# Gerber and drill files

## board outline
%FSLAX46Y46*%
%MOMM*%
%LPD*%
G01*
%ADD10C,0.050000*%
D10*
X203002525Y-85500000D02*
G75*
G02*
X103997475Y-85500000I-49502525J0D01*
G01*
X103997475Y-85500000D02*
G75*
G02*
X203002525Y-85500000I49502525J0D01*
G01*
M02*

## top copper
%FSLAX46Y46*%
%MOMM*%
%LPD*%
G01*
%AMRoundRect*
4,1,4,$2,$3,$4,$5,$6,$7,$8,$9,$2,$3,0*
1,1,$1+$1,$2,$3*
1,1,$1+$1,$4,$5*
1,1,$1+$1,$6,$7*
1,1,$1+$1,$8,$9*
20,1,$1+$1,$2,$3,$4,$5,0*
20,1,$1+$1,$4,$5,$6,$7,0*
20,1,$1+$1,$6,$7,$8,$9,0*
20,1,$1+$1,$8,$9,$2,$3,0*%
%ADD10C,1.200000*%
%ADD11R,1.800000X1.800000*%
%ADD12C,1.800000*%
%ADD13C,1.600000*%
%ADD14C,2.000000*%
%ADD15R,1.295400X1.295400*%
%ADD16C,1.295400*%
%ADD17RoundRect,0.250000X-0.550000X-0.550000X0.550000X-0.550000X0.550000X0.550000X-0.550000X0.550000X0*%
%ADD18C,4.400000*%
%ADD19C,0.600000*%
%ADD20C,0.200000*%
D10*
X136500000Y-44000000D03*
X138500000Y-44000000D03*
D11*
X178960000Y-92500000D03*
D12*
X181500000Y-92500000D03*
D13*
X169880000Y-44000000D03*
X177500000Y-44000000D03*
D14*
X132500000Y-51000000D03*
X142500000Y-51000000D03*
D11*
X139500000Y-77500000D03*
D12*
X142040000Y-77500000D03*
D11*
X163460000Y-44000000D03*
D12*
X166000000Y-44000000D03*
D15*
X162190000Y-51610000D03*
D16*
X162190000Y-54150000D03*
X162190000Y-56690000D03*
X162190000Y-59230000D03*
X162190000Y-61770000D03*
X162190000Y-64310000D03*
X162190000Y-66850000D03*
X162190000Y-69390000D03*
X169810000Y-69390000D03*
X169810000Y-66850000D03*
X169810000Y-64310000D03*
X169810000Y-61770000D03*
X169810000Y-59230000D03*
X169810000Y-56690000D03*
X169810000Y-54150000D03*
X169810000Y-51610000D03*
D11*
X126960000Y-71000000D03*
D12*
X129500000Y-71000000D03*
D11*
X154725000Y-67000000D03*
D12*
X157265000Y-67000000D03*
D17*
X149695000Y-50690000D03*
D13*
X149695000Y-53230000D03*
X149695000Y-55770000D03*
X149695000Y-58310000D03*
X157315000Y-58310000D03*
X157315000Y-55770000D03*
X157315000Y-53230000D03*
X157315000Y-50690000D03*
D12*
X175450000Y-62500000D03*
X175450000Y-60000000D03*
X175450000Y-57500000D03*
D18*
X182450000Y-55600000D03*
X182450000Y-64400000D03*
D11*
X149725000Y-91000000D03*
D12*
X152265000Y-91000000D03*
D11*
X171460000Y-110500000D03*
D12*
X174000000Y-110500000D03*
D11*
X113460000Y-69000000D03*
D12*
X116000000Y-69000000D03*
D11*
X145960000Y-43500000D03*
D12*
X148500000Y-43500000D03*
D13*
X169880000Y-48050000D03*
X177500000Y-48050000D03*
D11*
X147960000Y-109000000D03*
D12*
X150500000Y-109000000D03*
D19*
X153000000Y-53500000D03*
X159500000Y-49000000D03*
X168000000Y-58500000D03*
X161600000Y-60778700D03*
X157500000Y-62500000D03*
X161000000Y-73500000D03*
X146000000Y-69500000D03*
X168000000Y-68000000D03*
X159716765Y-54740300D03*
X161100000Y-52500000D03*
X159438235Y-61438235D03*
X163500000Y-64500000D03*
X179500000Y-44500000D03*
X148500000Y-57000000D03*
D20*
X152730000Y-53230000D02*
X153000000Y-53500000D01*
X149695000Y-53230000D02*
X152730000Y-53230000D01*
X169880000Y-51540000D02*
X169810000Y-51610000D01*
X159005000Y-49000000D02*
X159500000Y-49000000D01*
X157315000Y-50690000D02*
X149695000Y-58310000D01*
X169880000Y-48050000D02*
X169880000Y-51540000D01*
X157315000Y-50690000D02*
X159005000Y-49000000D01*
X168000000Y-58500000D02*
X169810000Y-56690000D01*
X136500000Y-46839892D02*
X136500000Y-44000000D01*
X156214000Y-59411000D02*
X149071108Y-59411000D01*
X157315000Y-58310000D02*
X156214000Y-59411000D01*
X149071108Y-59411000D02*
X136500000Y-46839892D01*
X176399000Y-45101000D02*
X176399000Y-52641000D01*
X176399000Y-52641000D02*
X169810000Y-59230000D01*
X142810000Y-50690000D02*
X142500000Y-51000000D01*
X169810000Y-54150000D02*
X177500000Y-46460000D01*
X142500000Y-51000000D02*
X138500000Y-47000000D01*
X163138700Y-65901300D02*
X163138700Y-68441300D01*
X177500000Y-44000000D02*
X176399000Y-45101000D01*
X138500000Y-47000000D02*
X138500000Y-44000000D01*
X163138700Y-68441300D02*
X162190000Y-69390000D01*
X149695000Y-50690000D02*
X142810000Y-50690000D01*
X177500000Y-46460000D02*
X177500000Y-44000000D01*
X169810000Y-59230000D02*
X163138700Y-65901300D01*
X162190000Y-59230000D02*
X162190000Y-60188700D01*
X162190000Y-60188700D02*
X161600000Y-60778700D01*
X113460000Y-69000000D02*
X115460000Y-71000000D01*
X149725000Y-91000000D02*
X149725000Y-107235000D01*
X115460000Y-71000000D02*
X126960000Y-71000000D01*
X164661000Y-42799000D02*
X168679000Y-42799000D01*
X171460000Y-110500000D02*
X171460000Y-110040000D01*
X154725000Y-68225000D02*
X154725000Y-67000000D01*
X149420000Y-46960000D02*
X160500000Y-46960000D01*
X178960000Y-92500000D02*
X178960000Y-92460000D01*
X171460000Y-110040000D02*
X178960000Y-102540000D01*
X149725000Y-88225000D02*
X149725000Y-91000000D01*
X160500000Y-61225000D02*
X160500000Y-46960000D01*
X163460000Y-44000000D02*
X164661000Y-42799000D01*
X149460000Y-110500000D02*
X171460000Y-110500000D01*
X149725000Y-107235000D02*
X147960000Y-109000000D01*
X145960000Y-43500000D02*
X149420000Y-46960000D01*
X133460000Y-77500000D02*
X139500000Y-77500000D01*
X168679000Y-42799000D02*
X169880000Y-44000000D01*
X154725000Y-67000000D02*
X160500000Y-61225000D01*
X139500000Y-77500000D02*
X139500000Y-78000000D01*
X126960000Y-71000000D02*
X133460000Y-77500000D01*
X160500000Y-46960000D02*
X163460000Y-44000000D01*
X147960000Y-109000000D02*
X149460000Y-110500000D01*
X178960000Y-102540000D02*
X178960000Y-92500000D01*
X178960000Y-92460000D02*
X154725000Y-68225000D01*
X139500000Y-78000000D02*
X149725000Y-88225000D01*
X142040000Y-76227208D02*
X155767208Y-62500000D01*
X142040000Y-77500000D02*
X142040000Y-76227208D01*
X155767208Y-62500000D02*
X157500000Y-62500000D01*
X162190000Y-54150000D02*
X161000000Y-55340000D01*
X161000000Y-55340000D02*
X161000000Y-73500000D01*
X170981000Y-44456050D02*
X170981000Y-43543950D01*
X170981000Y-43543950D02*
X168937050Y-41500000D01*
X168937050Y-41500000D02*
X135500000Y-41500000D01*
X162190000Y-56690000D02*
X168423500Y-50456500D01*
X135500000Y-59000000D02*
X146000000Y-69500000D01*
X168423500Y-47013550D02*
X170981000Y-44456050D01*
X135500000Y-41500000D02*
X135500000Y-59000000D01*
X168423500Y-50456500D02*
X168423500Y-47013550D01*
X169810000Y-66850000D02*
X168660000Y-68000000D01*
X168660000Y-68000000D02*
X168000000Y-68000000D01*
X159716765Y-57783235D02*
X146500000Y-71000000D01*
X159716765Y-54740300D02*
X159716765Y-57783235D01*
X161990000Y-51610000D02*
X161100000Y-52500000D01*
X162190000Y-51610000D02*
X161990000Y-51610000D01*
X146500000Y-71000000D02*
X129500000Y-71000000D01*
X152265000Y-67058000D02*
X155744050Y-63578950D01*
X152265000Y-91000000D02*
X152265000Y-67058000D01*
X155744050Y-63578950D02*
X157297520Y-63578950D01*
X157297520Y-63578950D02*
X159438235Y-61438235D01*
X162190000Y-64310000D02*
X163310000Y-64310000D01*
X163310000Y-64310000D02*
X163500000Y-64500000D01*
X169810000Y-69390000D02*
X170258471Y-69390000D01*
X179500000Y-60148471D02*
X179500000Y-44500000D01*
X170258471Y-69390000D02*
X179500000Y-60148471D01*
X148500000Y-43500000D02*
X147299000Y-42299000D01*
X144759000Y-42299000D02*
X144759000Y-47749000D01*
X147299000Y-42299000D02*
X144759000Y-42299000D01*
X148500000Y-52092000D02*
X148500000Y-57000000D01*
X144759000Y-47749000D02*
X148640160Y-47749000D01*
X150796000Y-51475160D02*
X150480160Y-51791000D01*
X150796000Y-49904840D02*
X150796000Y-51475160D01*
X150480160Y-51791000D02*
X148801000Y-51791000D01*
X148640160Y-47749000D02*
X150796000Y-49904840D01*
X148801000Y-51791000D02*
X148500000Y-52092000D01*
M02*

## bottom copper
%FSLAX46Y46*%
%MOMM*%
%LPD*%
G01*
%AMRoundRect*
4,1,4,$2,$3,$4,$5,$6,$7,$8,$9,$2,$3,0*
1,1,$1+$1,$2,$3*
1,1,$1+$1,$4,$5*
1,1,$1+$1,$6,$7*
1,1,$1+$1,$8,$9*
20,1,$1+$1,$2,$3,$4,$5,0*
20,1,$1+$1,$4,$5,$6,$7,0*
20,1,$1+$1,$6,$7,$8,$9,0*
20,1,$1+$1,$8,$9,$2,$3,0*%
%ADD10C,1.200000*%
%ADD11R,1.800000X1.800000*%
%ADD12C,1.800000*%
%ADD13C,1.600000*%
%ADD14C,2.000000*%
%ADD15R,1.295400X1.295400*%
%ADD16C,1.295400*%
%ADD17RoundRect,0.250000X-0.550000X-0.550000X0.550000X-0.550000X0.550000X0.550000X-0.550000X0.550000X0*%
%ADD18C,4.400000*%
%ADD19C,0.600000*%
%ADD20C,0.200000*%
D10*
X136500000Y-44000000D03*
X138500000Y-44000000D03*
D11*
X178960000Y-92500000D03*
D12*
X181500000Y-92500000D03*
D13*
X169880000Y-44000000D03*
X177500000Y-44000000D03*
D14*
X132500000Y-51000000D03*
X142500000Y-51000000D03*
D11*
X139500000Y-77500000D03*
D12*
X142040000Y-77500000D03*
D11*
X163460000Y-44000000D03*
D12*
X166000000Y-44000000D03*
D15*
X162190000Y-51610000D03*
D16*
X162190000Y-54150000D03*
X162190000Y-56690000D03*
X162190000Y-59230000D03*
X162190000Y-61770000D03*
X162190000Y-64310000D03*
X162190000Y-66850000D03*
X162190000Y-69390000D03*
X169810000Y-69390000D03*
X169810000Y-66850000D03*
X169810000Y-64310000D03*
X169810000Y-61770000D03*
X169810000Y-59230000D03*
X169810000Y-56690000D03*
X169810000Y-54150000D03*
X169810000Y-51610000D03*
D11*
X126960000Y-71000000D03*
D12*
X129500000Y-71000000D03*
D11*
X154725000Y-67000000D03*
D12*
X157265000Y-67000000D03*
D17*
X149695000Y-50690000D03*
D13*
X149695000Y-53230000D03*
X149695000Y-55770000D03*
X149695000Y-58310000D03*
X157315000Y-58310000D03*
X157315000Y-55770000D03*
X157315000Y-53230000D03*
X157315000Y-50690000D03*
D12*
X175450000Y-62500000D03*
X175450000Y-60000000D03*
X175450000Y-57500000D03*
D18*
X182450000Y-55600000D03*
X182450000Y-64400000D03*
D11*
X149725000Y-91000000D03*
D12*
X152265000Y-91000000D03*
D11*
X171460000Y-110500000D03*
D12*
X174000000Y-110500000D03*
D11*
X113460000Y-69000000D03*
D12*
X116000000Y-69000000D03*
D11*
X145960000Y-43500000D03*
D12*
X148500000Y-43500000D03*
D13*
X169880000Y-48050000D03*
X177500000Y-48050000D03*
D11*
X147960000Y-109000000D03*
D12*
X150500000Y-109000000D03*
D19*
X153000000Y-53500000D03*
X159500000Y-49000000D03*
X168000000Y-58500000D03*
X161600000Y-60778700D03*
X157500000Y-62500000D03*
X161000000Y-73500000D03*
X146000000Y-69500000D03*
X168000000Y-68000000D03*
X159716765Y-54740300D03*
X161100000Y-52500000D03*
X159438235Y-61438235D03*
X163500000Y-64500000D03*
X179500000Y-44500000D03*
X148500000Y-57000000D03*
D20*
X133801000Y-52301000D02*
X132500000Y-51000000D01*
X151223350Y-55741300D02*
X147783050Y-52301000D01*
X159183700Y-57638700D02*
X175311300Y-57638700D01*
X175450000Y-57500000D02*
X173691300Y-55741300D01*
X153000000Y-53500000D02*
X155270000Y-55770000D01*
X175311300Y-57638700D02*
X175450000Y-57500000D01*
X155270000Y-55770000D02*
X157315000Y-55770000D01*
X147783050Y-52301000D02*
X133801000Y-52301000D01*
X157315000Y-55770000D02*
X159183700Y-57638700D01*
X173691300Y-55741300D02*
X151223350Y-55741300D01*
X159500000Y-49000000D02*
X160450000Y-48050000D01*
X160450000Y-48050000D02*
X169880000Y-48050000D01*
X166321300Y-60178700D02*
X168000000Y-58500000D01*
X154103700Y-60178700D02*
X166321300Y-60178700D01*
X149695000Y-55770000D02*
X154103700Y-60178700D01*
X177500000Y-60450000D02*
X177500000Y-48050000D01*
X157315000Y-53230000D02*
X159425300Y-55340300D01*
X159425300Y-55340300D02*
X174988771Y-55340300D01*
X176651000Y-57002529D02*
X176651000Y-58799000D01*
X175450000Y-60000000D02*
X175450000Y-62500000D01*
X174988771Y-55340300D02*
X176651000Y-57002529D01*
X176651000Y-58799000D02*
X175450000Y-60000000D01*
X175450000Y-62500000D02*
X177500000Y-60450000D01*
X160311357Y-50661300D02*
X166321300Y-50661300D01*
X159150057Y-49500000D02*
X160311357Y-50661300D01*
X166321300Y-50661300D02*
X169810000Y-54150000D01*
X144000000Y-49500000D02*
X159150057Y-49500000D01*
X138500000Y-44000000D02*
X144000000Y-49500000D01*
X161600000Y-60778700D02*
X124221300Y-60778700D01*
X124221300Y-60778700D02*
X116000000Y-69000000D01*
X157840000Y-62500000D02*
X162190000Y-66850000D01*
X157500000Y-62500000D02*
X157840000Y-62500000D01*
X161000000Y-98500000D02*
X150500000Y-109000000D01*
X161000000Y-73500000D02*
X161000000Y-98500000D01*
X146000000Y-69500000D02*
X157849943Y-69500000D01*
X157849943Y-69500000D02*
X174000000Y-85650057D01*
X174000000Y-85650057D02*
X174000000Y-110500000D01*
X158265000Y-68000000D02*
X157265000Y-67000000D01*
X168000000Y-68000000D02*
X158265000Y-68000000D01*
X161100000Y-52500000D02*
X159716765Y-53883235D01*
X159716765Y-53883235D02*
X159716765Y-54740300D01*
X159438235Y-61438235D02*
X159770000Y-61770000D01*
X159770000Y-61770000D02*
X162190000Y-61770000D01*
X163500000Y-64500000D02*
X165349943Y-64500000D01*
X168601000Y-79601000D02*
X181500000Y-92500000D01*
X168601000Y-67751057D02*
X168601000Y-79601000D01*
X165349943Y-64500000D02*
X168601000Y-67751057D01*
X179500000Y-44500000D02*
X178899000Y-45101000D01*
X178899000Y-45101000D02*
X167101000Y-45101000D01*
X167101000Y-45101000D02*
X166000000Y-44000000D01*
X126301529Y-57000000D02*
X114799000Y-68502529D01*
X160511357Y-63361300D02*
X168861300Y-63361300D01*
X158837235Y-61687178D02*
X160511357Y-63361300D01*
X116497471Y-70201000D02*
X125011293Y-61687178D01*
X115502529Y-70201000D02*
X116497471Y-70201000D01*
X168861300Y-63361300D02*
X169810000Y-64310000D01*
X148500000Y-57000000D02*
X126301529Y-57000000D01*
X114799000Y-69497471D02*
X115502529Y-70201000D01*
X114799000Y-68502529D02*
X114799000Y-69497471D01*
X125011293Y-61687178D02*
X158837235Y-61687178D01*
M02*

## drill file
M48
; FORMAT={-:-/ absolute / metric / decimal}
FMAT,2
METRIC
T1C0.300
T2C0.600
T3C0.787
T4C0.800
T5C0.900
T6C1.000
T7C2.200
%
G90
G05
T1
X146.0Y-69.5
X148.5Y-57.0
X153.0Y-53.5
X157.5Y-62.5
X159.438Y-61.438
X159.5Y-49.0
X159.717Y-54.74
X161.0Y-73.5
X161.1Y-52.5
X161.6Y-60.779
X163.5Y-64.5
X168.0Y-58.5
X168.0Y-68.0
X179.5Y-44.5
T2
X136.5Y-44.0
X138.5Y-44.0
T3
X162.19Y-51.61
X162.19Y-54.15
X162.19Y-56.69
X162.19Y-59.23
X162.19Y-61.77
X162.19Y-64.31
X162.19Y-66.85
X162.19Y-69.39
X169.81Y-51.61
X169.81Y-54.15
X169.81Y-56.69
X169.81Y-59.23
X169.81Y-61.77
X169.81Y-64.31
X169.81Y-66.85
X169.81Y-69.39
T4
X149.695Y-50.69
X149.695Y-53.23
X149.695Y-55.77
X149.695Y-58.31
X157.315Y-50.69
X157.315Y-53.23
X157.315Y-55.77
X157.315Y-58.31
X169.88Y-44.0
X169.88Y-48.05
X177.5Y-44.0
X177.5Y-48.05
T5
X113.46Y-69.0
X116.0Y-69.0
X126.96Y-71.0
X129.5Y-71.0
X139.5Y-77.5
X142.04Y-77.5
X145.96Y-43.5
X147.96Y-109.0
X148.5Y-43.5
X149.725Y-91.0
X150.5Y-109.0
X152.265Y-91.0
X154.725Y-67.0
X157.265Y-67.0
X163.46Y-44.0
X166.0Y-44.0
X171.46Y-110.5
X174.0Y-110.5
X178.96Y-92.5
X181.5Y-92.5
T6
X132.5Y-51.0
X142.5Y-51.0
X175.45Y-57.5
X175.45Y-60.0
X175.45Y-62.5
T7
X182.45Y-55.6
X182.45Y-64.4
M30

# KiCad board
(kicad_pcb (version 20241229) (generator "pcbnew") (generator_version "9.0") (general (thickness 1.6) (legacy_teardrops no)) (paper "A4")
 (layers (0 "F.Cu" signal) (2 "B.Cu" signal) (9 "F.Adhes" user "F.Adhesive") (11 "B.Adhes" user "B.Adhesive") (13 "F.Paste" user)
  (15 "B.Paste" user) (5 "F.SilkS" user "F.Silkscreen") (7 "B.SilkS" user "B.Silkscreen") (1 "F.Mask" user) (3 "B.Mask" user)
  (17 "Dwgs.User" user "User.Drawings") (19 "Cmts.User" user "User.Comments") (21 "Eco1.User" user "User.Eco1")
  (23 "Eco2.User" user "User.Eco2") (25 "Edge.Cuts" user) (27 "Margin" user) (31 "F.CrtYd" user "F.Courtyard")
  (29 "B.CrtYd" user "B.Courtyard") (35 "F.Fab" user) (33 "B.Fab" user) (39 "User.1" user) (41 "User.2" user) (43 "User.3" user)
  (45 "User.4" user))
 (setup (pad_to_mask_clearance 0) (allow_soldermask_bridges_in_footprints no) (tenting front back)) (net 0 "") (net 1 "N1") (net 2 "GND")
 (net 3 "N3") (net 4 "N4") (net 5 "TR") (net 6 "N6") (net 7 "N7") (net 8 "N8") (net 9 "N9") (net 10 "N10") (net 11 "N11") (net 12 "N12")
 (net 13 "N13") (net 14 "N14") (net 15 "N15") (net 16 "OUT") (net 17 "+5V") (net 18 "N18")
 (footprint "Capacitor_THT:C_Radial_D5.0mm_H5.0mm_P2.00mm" (layer "F.Cu") (at 136.5 44)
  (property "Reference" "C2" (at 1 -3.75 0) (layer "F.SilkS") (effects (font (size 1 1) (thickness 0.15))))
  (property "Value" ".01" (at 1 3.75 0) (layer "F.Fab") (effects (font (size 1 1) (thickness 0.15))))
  (pad "1" thru_hole circle (at 0 0) (size 1.2 1.2) (drill 0.6) (layers "*.Cu" "*.Mask") (remove_unused_layers no) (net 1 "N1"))
  (pad "2" thru_hole circle (at 2 0) (size 1.2 1.2) (drill 0.6) (layers "*.Cu" "*.Mask") (remove_unused_layers no) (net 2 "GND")))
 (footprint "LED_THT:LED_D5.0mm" (layer "F.Cu") (at 178.96 92.5)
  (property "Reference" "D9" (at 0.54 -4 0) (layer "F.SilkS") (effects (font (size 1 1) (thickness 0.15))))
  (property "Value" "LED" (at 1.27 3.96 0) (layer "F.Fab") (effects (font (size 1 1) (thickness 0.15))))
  (pad "1" thru_hole rect (at 0 0) (size 1.8 1.8) (drill 0.9) (layers "*.Cu" "*.Mask") (remove_unused_layers no) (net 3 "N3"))
  (pad "2" thru_hole circle (at 2.54 0) (size 1.8 1.8) (drill 0.9) (layers "*.Cu" "*.Mask") (remove_unused_layers no) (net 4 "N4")))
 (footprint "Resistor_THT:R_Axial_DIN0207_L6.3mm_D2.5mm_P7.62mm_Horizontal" (layer "F.Cu") (at 169.88 44)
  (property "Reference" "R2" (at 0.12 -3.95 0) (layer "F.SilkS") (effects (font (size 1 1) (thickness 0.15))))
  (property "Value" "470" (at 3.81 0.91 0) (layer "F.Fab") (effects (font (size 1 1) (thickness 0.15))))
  (pad "1" thru_hole circle (at 0 0) (size 1.6 1.6) (drill 0.8) (layers "*.Cu" "*.Mask") (remove_unused_layers no) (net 3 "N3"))
  (pad "2" thru_hole circle (at 7.62 0) (size 1.6 1.6) (drill 0.8) (layers "*.Cu" "*.Mask") (remove_unused_layers no) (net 2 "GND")))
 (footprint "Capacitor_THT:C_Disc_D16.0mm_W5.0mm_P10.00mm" (layer "F.Cu") (at 132.5 51)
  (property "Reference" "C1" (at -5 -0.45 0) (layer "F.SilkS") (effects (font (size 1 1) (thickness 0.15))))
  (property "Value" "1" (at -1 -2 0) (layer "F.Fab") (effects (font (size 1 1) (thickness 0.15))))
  (pad "1" thru_hole circle (at 0 0) (size 2 2) (drill 1) (layers "*.Cu" "*.Mask") (remove_unused_layers no) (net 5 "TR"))
  (pad "2" thru_hole circle (at 10 0) (size 2 2) (drill 1) (layers "*.Cu" "*.Mask") (remove_unused_layers no) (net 2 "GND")))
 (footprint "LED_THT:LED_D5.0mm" (layer "F.Cu") (at 139.5 77.5)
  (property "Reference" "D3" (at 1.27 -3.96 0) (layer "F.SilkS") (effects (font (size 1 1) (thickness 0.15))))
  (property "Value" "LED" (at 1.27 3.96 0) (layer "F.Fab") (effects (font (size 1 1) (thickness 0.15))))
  (pad "1" thru_hole rect (at 0 0) (size 1.8 1.8) (drill 0.9) (layers "*.Cu" "*.Mask") (remove_unused_layers no) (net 3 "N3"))
  (pad "2" thru_hole circle (at 2.54 0) (size 1.8 1.8) (drill 0.9) (layers "*.Cu" "*.Mask") (remove_unused_layers no) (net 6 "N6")))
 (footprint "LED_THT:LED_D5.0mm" (layer "F.Cu") (at 163.46 44)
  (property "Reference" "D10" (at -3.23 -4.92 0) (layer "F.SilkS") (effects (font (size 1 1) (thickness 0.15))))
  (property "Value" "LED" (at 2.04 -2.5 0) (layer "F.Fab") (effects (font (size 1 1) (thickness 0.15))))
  (pad "1" thru_hole rect (at 0 0) (size 1.8 1.8) (drill 0.9) (layers "*.Cu" "*.Mask") (remove_unused_layers no) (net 3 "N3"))
  (pad "2" thru_hole circle (at 2.54 0) (size 1.8 1.8) (drill 0.9) (layers "*.Cu" "*.Mask") (remove_unused_layers no) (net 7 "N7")))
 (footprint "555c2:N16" (layer "F.Cu") (at 169.81 69.39)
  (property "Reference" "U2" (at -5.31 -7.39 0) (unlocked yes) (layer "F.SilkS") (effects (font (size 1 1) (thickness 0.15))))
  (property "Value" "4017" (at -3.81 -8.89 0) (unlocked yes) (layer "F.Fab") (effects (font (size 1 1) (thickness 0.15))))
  (pad "1" thru_hole rect (at -7.62 -17.78) (size 1.2954 1.2954) (drill 0.7874) (layers "*.Cu" "*.Mask") (remove_unused_layers no)
   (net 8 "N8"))
  (pad "2" thru_hole circle (at -7.62 -15.24) (size 1.2954 1.2954) (drill 0.7874) (layers "*.Cu" "*.Mask") (remove_unused_layers no)
   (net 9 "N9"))
  (pad "3" thru_hole circle (at -7.62 -12.7) (size 1.2954 1.2954) (drill 0.7874) (layers "*.Cu" "*.Mask") (remove_unused_layers no)
   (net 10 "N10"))
  (pad "4" thru_hole circle (at -7.62 -10.16) (size 1.2954 1.2954) (drill 0.7874) (layers "*.Cu" "*.Mask") (remove_unused_layers no)
   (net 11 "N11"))
  (pad "5" thru_hole circle (at -7.62 -7.62) (size 1.2954 1.2954) (drill 0.7874) (layers "*.Cu" "*.Mask") (remove_unused_layers no)
   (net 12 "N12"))
  (pad "6" thru_hole circle (at -7.62 -5.08) (size 1.2954 1.2954) (drill 0.7874) (layers "*.Cu" "*.Mask") (remove_unused_layers no)
   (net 4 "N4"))
  (pad "7" thru_hole circle (at -7.62 -2.54) (size 1.2954 1.2954) (drill 0.7874) (layers "*.Cu" "*.Mask") (remove_unused_layers no)
   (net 6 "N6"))
  (pad "8" thru_hole circle (at -7.62 0) (size 1.2954 1.2954) (drill 0.7874) (layers "*.Cu" "*.Mask") (remove_unused_layers no)
   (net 2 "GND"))
  (pad "9" thru_hole circle (at 0 0) (size 1.2954 1.2954) (drill 0.7874) (layers "*.Cu" "*.Mask") (remove_unused_layers no) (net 7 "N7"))
  (pad "10" thru_hole circle (at 0 -2.54) (size 1.2954 1.2954) (drill 0.7874) (layers "*.Cu" "*.Mask") (remove_unused_layers no)
   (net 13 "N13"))
  (pad "11" thru_hole circle (at 0 -5.08) (size 1.2954 1.2954) (drill 0.7874) (layers "*.Cu" "*.Mask") (remove_unused_layers no)
   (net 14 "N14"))
  (pad "12" thru_hole circle (at 0 -7.62) (size 1.2954 1.2954) (drill 0.7874) (layers "*.Cu" "*.Mask") (remove_unused_layers no)
   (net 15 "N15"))
  (pad "13" thru_hole circle (at 0 -10.16) (size 1.2954 1.2954) (drill 0.7874) (layers "*.Cu" "*.Mask") (remove_unused_layers no)
   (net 2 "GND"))
  (pad "14" thru_hole circle (at 0 -12.7) (size 1.2954 1.2954) (drill 0.7874) (layers "*.Cu" "*.Mask") (remove_unused_layers no)
   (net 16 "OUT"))
  (pad "15" thru_hole circle (at 0 -15.24) (size 1.2954 1.2954) (drill 0.7874) (layers "*.Cu" "*.Mask") (remove_unused_layers no)
   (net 2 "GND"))
  (pad "16" thru_hole circle (at 0 -17.78) (size 1.2954 1.2954) (drill 0.7874) (layers "*.Cu" "*.Mask") (remove_unused_layers no)
   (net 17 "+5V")))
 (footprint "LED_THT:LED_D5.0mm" (layer "F.Cu") (at 126.96 71)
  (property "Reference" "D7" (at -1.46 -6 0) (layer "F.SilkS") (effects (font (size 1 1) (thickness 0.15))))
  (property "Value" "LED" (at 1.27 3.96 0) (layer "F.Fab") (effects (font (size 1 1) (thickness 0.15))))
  (pad "1" thru_hole rect (at 0 0) (size 1.8 1.8) (drill 0.9) (layers "*.Cu" "*.Mask") (remove_unused_layers no) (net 3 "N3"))
  (pad "2" thru_hole circle (at 2.54 0) (size 1.8 1.8) (drill 0.9) (layers "*.Cu" "*.Mask") (remove_unused_layers no) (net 8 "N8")))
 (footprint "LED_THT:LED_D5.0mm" (layer "F.Cu") (at 154.725 67)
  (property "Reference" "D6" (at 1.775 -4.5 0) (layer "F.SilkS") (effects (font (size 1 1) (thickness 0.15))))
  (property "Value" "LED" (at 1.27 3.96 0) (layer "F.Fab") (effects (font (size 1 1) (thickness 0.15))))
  (pad "1" thru_hole rect (at 0 0) (size 1.8 1.8) (drill 0.9) (layers "*.Cu" "*.Mask") (remove_unused_layers no) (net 3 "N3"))
  (pad "2" thru_hole circle (at 2.54 0) (size 1.8 1.8) (drill 0.9) (layers "*.Cu" "*.Mask") (remove_unused_layers no) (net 13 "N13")))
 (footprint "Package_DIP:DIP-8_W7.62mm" (layer "F.Cu") (at 149.695 50.69)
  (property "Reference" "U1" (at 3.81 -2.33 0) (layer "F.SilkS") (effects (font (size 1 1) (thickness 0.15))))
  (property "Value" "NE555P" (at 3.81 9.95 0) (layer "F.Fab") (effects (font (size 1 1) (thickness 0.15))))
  (pad "1" thru_hole roundrect (at 0 0) (size 1.6 1.6) (drill 0.8) (layers "*.Cu" "*.Mask") (remove_unused_layers no)
   (roundrect_rratio 0.15625) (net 2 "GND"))
  (pad "2" thru_hole circle (at 0 2.54) (size 1.6 1.6) (drill 0.8) (layers "*.Cu" "*.Mask") (remove_unused_layers no) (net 5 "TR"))
  (pad "3" thru_hole circle (at 0 5.08) (size 1.6 1.6) (drill 0.8) (layers "*.Cu" "*.Mask") (remove_unused_layers no) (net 16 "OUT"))
  (pad "4" thru_hole circle (at 0 7.62) (size 1.6 1.6) (drill 0.8) (layers "*.Cu" "*.Mask") (remove_unused_layers no) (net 17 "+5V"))
  (pad "5" thru_hole circle (at 7.62 7.62) (size 1.6 1.6) (drill 0.8) (layers "*.Cu" "*.Mask") (remove_unused_layers no) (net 1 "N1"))
  (pad "6" thru_hole circle (at 7.62 5.08) (size 1.6 1.6) (drill 0.8) (layers "*.Cu" "*.Mask") (remove_unused_layers no) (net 5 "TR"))
  (pad "7" thru_hole circle (at 7.62 2.54) (size 1.6 1.6) (drill 0.8) (layers "*.Cu" "*.Mask") (remove_unused_layers no) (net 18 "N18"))
  (pad "8" thru_hole circle (at 7.62 0) (size 1.6 1.6) (drill 0.8) (layers "*.Cu" "*.Mask") (remove_unused_layers no) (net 17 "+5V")))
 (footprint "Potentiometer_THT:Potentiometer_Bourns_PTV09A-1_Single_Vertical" (layer "F.Cu") (at 175.45 62.5)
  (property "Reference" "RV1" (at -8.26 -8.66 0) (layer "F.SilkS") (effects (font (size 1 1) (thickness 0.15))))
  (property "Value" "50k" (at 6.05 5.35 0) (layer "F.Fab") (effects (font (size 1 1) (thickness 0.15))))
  (pad "1" thru_hole circle (at 0 0) (size 1.8 1.8) (drill 1) (layers "*.Cu" "*.Mask") (remove_unused_layers no) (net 18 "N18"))
  (pad "2" thru_hole circle (at 0 -2.5) (size 1.8 1.8) (drill 1) (layers "*.Cu" "*.Mask") (remove_unused_layers no) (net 18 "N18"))
  (pad "3" thru_hole circle (at 0 -5) (size 1.8 1.8) (drill 1) (layers "*.Cu" "*.Mask") (remove_unused_layers no) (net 5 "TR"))
  (pad "MP" thru_hole circle (at 7 -6.9) (size 4.4 4.4) (drill 2.2) (layers "*.Cu" "*.Mask") (remove_unused_layers no))
  (pad "MP" thru_hole circle (at 7 1.9) (size 4.4 4.4) (drill 2.2) (layers "*.Cu" "*.Mask") (remove_unused_layers no)))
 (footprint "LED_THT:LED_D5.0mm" (layer "F.Cu") (at 149.725 91)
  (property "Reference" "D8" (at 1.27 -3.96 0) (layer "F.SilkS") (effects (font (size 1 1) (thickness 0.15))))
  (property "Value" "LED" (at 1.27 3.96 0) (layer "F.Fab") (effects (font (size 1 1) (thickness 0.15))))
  (pad "1" thru_hole rect (at 0 0) (size 1.8 1.8) (drill 0.9) (layers "*.Cu" "*.Mask") (remove_unused_layers no) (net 3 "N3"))
  (pad "2" thru_hole circle (at 2.54 0) (size 1.8 1.8) (drill 0.9) (layers "*.Cu" "*.Mask") (remove_unused_layers no) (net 12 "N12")))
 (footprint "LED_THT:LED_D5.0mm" (layer "F.Cu") (at 171.46 110.5)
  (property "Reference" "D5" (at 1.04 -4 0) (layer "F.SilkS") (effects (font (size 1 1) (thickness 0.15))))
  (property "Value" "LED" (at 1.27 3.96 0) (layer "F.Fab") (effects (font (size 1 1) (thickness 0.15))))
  (pad "1" thru_hole rect (at 0 0) (size 1.8 1.8) (drill 0.9) (layers "*.Cu" "*.Mask") (remove_unused_layers no) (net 3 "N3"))
  (pad "2" thru_hole circle (at 2.54 0) (size 1.8 1.8) (drill 0.9) (layers "*.Cu" "*.Mask") (remove_unused_layers no) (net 10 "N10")))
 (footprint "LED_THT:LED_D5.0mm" (layer "F.Cu") (at 113.46 69)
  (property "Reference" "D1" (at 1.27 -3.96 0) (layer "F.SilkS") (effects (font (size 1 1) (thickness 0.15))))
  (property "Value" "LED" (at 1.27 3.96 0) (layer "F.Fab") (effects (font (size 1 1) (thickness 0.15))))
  (pad "1" thru_hole rect (at 0 0) (size 1.8 1.8) (drill 0.9) (layers "*.Cu" "*.Mask") (remove_unused_layers no) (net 3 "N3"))
  (pad "2" thru_hole circle (at 2.54 0) (size 1.8 1.8) (drill 0.9) (layers "*.Cu" "*.Mask") (remove_unused_layers no) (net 11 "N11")))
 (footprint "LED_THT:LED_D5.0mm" (layer "F.Cu") (at 145.96 43.5)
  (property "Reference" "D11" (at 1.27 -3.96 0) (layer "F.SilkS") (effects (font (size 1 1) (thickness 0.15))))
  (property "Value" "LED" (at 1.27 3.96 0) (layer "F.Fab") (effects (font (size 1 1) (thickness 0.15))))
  (pad "1" thru_hole rect (at 0 0) (size 1.8 1.8) (drill 0.9) (layers "*.Cu" "*.Mask") (remove_unused_layers no) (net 3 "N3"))
  (pad "2" thru_hole circle (at 2.54 0) (size 1.8 1.8) (drill 0.9) (layers "*.Cu" "*.Mask") (remove_unused_layers no) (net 14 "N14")))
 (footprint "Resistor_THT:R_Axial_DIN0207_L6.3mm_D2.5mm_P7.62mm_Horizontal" (layer "F.Cu") (at 169.88 48.05)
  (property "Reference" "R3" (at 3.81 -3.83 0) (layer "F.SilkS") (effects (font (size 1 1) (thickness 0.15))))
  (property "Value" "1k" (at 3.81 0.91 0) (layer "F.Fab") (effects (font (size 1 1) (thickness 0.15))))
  (pad "1" thru_hole circle (at 0 0) (size 1.6 1.6) (drill 0.8) (layers "*.Cu" "*.Mask") (remove_unused_layers no) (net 17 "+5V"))
  (pad "2" thru_hole circle (at 7.62 0) (size 1.6 1.6) (drill 0.8) (layers "*.Cu" "*.Mask") (remove_unused_layers no) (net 18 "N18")))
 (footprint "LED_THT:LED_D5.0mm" (layer "F.Cu") (at 147.96 109)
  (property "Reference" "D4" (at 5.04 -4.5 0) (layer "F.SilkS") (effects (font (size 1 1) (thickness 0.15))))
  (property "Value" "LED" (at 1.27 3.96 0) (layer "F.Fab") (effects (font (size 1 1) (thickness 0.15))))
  (pad "1" thru_hole rect (at 0 0) (size 1.8 1.8) (drill 0.9) (layers "*.Cu" "*.Mask") (remove_unused_layers no) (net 3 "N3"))
  (pad "2" thru_hole circle (at 2.54 0) (size 1.8 1.8) (drill 0.9) (layers "*.Cu" "*.Mask") (remove_unused_layers no) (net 9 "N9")))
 (gr_circle (center 153.5 85.5) (end 119 50) (stroke (width 0.05) (type default)) (fill no) (layer "Edge.Cuts"))
 (segment (start 152.73 53.23) (end 153 53.5) (width 0.2) (layer "F.Cu") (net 5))
 (segment (start 149.695 53.23) (end 152.73 53.23) (width 0.2) (layer "F.Cu") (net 5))
 (via (at 153 53.5) (size 0.6) (drill 0.3) (layers "F.Cu" "B.Cu") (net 5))
 (segment (start 133.801 52.301) (end 132.5 51) (width 0.2) (layer "B.Cu") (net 5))
 (segment (start 151.22335 55.7413) (end 147.78305 52.301) (width 0.2) (layer "B.Cu") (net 5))
 (segment (start 159.1837 57.6387) (end 175.3113 57.6387) (width 0.2) (layer "B.Cu") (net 5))
 (segment (start 175.45 57.5) (end 173.6913 55.7413) (width 0.2) (layer "B.Cu") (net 5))
 (segment (start 153 53.5) (end 155.27 55.77) (width 0.2) (layer "B.Cu") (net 5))
 (segment (start 175.3113 57.6387) (end 175.45 57.5) (width 0.2) (layer "B.Cu") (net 5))
 (segment (start 155.27 55.77) (end 157.315 55.77) (width 0.2) (layer "B.Cu") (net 5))
 (segment (start 147.78305 52.301) (end 133.801 52.301) (width 0.2) (layer "B.Cu") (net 5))
 (segment (start 157.315 55.77) (end 159.1837 57.6387) (width 0.2) (layer "B.Cu") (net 5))
 (segment (start 173.6913 55.7413) (end 151.22335 55.7413) (width 0.2) (layer "B.Cu") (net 5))
 (segment (start 169.88 51.54) (end 169.81 51.61) (width 0.2) (layer "F.Cu") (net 17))
 (segment (start 159.005 49) (end 159.5 49) (width 0.2) (layer "F.Cu") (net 17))
 (segment (start 157.315 50.69) (end 149.695 58.31) (width 0.2) (layer "F.Cu") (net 17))
 (segment (start 169.88 48.05) (end 169.88 51.54) (width 0.2) (layer "F.Cu") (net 17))
 (segment (start 157.315 50.69) (end 159.005 49) (width 0.2) (layer "F.Cu") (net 17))
 (via (at 159.5 49) (size 0.6) (drill 0.3) (layers "F.Cu" "B.Cu") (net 17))
 (segment (start 159.5 49) (end 160.45 48.05) (width 0.2) (layer "B.Cu") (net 17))
 (segment (start 160.45 48.05) (end 169.88 48.05) (width 0.2) (layer "B.Cu") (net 17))
 (segment (start 168 58.5) (end 169.81 56.69) (width 0.2) (layer "F.Cu") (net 16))
 (via (at 168 58.5) (size 0.6) (drill 0.3) (layers "F.Cu" "B.Cu") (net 16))
 (segment (start 166.3213 60.1787) (end 168 58.5) (width 0.2) (layer "B.Cu") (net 16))
 (segment (start 154.1037 60.1787) (end 166.3213 60.1787) (width 0.2) (layer "B.Cu") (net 16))
 (segment (start 149.695 55.77) (end 154.1037 60.1787) (width 0.2) (layer "B.Cu") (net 16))
 (segment (start 136.5 46.839892) (end 136.5 44) (width 0.2) (layer "F.Cu") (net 1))
 (segment (start 156.214 59.411) (end 149.071108 59.411) (width 0.2) (layer "F.Cu") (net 1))
 (segment (start 157.315 58.31) (end 156.214 59.411) (width 0.2) (layer "F.Cu") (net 1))
 (segment (start 149.071108 59.411) (end 136.5 46.839892) (width 0.2) (layer "F.Cu") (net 1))
 (segment (start 177.5 60.45) (end 177.5 48.05) (width 0.2) (layer "B.Cu") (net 18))
 (segment (start 157.315 53.23) (end 159.4253 55.3403) (width 0.2) (layer "B.Cu") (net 18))
 (segment (start 159.4253 55.3403) (end 174.988771 55.3403) (width 0.2) (layer "B.Cu") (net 18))
 (segment (start 176.651 57.002529) (end 176.651 58.799) (width 0.2) (layer "B.Cu") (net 18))
 (segment (start 175.45 60) (end 175.45 62.5) (width 0.2) (layer "B.Cu") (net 18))
 (segment (start 174.988771 55.3403) (end 176.651 57.002529) (width 0.2) (layer "B.Cu") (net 18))
 (segment (start 176.651 58.799) (end 175.45 60) (width 0.2) (layer "B.Cu") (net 18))
 (segment (start 175.45 62.5) (end 177.5 60.45) (width 0.2) (layer "B.Cu") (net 18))
 (segment (start 176.399 45.101) (end 176.399 52.641) (width 0.2) (layer "F.Cu") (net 2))
 (segment (start 176.399 52.641) (end 169.81 59.23) (width 0.2) (layer "F.Cu") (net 2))
 (segment (start 142.81 50.69) (end 142.5 51) (width 0.2) (layer "F.Cu") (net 2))
 (segment (start 169.81 54.15) (end 177.5 46.46) (width 0.2) (layer "F.Cu") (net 2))
 (segment (start 142.5 51) (end 138.5 47) (width 0.2) (layer "F.Cu") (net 2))
 (segment (start 163.1387 65.9013) (end 163.1387 68.4413) (width 0.2) (layer "F.Cu") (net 2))
 (segment (start 177.5 44) (end 176.399 45.101) (width 0.2) (layer "F.Cu") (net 2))
 (segment (start 138.5 47) (end 138.5 44) (width 0.2) (layer "F.Cu") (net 2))
 (segment (start 163.1387 68.4413) (end 162.19 69.39) (width 0.2) (layer "F.Cu") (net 2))
 (segment (start 149.695 50.69) (end 142.81 50.69) (width 0.2) (layer "F.Cu") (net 2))
 (segment (start 177.5 46.46) (end 177.5 44) (width 0.2) (layer "F.Cu") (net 2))
 (segment (start 169.81 59.23) (end 163.1387 65.9013) (width 0.2) (layer "F.Cu") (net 2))
 (segment (start 160.311357 50.6613) (end 166.3213 50.6613) (width 0.2) (layer "B.Cu") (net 2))
 (segment (start 159.150057 49.5) (end 160.311357 50.6613) (width 0.2) (layer "B.Cu") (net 2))
 (segment (start 166.3213 50.6613) (end 169.81 54.15) (width 0.2) (layer "B.Cu") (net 2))
 (segment (start 144 49.5) (end 159.150057 49.5) (width 0.2) (layer "B.Cu") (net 2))
 (segment (start 138.5 44) (end 144 49.5) (width 0.2) (layer "B.Cu") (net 2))
 (segment (start 162.19 59.23) (end 162.19 60.1887) (width 0.2) (layer "F.Cu") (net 11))
 (segment (start 162.19 60.1887) (end 161.6 60.7787) (width 0.2) (layer "F.Cu") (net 11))
 (via (at 161.6 60.7787) (size 0.6) (drill 0.3) (layers "F.Cu" "B.Cu") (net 11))
 (segment (start 161.6 60.7787) (end 124.2213 60.7787) (width 0.2) (layer "B.Cu") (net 11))
 (segment (start 124.2213 60.7787) (end 116 69) (width 0.2) (layer "B.Cu") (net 11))
 (segment (start 113.46 69) (end 115.46 71) (width 0.2) (layer "F.Cu") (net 3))
 (segment (start 149.725 91) (end 149.725 107.235) (width 0.2) (layer "F.Cu") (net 3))
 (segment (start 115.46 71) (end 126.96 71) (width 0.2) (layer "F.Cu") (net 3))
 (segment (start 164.661 42.799) (end 168.679 42.799) (width 0.2) (layer "F.Cu") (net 3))
 (segment (start 171.46 110.5) (end 171.46 110.04) (width 0.2) (layer "F.Cu") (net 3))
 (segment (start 154.725 68.225) (end 154.725 67) (width 0.2) (layer "F.Cu") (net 3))
 (segment (start 149.42 46.96) (end 160.5 46.96) (width 0.2) (layer "F.Cu") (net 3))
 (segment (start 178.96 92.5) (end 178.96 92.46) (width 0.2) (layer "F.Cu") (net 3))
 (segment (start 171.46 110.04) (end 178.96 102.54) (width 0.2) (layer "F.Cu") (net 3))
 (segment (start 149.725 88.225) (end 149.725 91) (width 0.2) (layer "F.Cu") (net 3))
 (segment (start 160.5 61.225) (end 160.5 46.96) (width 0.2) (layer "F.Cu") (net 3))
 (segment (start 163.46 44) (end 164.661 42.799) (width 0.2) (layer "F.Cu") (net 3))
 (segment (start 149.46 110.5) (end 171.46 110.5) (width 0.2) (layer "F.Cu") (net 3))
 (segment (start 149.725 107.235) (end 147.96 109) (width 0.2) (layer "F.Cu") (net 3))
 (segment (start 145.96 43.5) (end 149.42 46.96) (width 0.2) (layer "F.Cu") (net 3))
 (segment (start 133.46 77.5) (end 139.5 77.5) (width 0.2) (layer "F.Cu") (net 3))
 (segment (start 168.679 42.799) (end 169.88 44) (width 0.2) (layer "F.Cu") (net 3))
 (segment (start 154.725 67) (end 160.5 61.225) (width 0.2) (layer "F.Cu") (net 3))
 (segment (start 139.5 77.5) (end 139.5 78) (width 0.2) (layer "F.Cu") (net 3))
 (segment (start 126.96 71) (end 133.46 77.5) (width 0.2) (layer "F.Cu") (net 3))
 (segment (start 160.5 46.96) (end 163.46 44) (width 0.2) (layer "F.Cu") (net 3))
 (segment (start 147.96 109) (end 149.46 110.5) (width 0.2) (layer "F.Cu") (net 3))
 (segment (start 178.96 102.54) (end 178.96 92.5) (width 0.2) (layer "F.Cu") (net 3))
 (segment (start 178.96 92.46) (end 154.725 68.225) (width 0.2) (layer "F.Cu") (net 3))
 (segment (start 139.5 78) (end 149.725 88.225) (width 0.2) (layer "F.Cu") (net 3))
 (segment (start 142.04 76.227208) (end 155.767208 62.5) (width 0.2) (layer "F.Cu") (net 6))
 (segment (start 142.04 77.5) (end 142.04 76.227208) (width 0.2) (layer "F.Cu") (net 6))
 (segment (start 155.767208 62.5) (end 157.5 62.5) (width 0.2) (layer "F.Cu") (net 6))
 (via (at 157.5 62.5) (size 0.6) (drill 0.3) (layers "F.Cu" "B.Cu") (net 6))
 (segment (start 157.84 62.5) (end 162.19 66.85) (width 0.2) (layer "B.Cu") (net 6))
 (segment (start 157.5 62.5) (end 157.84 62.5) (width 0.2) (layer "B.Cu") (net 6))
 (segment (start 162.19 54.15) (end 161 55.34) (width 0.2) (layer "F.Cu") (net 9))
 (segment (start 161 55.34) (end 161 73.5) (width 0.2) (layer "F.Cu") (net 9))
 (via (at 161 73.5) (size 0.6) (drill 0.3) (layers "F.Cu" "B.Cu") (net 9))
 (segment (start 161 98.5) (end 150.5 109) (width 0.2) (layer "B.Cu") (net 9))
 (segment (start 161 73.5) (end 161 98.5) (width 0.2) (layer "B.Cu") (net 9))
 (segment (start 170.981 44.45605) (end 170.981 43.54395) (width 0.2) (layer "F.Cu") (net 10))
 (segment (start 170.981 43.54395) (end 168.93705 41.5) (width 0.2) (layer "F.Cu") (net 10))
 (segment (start 168.93705 41.5) (end 135.5 41.5) (width 0.2) (layer "F.Cu") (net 10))
 (segment (start 162.19 56.69) (end 168.4235 50.4565) (width 0.2) (layer "F.Cu") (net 10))
 (segment (start 135.5 59) (end 146 69.5) (width 0.2) (layer "F.Cu") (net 10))
 (segment (start 168.4235 47.01355) (end 170.981 44.45605) (width 0.2) (layer "F.Cu") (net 10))
 (segment (start 135.5 41.5) (end 135.5 59) (width 0.2) (layer "F.Cu") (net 10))
 (segment (start 168.4235 50.4565) (end 168.4235 47.01355) (width 0.2) (layer "F.Cu") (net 10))
 (via (at 146 69.5) (size 0.6) (drill 0.3) (layers "F.Cu" "B.Cu") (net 10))
 (segment (start 146 69.5) (end 157.849943 69.5) (width 0.2) (layer "B.Cu") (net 10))
 (segment (start 157.849943 69.5) (end 174 85.650057) (width 0.2) (layer "B.Cu") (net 10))
 (segment (start 174 85.650057) (end 174 110.5) (width 0.2) (layer "B.Cu") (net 10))
 (segment (start 169.81 66.85) (end 168.66 68) (width 0.2) (layer "F.Cu") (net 13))
 (segment (start 168.66 68) (end 168 68) (width 0.2) (layer "F.Cu") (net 13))
 (via (at 168 68) (size 0.6) (drill 0.3) (layers "F.Cu" "B.Cu") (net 13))
 (segment (start 158.265 68) (end 157.265 67) (width 0.2) (layer "B.Cu") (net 13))
 (segment (start 168 68) (end 158.265 68) (width 0.2) (layer "B.Cu") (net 13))
 (segment (start 159.716765 57.783235) (end 146.5 71) (width 0.2) (layer "F.Cu") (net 8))
 (segment (start 159.716765 54.7403) (end 159.716765 57.783235) (width 0.2) (layer "F.Cu") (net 8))
 (segment (start 161.99 51.61) (end 161.1 52.5) (width 0.2) (layer "F.Cu") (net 8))
 (segment (start 162.19 51.61) (end 161.99 51.61) (width 0.2) (layer "F.Cu") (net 8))
 (segment (start 146.5 71) (end 129.5 71) (width 0.2) (layer "F.Cu") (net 8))
 (via (at 159.716765 54.7403) (size 0.6) (drill 0.3) (layers "F.Cu" "B.Cu") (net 8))
 (via (at 161.1 52.5) (size 0.6) (drill 0.3) (layers "F.Cu" "B.Cu") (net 8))
 (segment (start 161.1 52.5) (end 159.716765 53.883235) (width 0.2) (layer "B.Cu") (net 8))
 (segment (start 159.716765 53.883235) (end 159.716765 54.7403) (width 0.2) (layer "B.Cu") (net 8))
 (segment (start 152.265 67.058) (end 155.74405 63.57895) (width 0.2) (layer "F.Cu") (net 12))
 (segment (start 152.265 91) (end 152.265 67.058) (width 0.2) (layer "F.Cu") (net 12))
 (segment (start 155.74405 63.57895) (end 157.29752 63.57895) (width 0.2) (layer "F.Cu") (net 12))
 (segment (start 157.29752 63.57895) (end 159.438235 61.438235) (width 0.2) (layer "F.Cu") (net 12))
 (via (at 159.438235 61.438235) (size 0.6) (drill 0.3) (layers "F.Cu" "B.Cu") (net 12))
 (segment (start 159.438235 61.438235) (end 159.77 61.77) (width 0.2) (layer "B.Cu") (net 12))
 (segment (start 159.77 61.77) (end 162.19 61.77) (width 0.2) (layer "B.Cu") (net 12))
 (segment (start 162.19 64.31) (end 163.31 64.31) (width 0.2) (layer "F.Cu") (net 4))
 (segment (start 163.31 64.31) (end 163.5 64.5) (width 0.2) (layer "F.Cu") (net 4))
 (via (at 163.5 64.5) (size 0.6) (drill 0.3) (layers "F.Cu" "B.Cu") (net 4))
 (segment (start 163.5 64.5) (end 165.349943 64.5) (width 0.2) (layer "B.Cu") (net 4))
 (segment (start 168.601 79.601) (end 181.5 92.5) (width 0.2) (layer "B.Cu") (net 4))
 (segment (start 168.601 67.751057) (end 168.601 79.601) (width 0.2) (layer "B.Cu") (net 4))
 (segment (start 165.349943 64.5) (end 168.601 67.751057) (width 0.2) (layer "B.Cu") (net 4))
 (segment (start 169.81 69.39) (end 170.258471 69.39) (width 0.2) (layer "F.Cu") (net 7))
 (segment (start 179.5 60.148471) (end 179.5 44.5) (width 0.2) (layer "F.Cu") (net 7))
 (segment (start 170.258471 69.39) (end 179.5 60.148471) (width 0.2) (layer "F.Cu") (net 7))
 (via (at 179.5 44.5) (size 0.6) (drill 0.3) (layers "F.Cu" "B.Cu") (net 7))
 (segment (start 179.5 44.5) (end 178.899 45.101) (width 0.2) (layer "B.Cu") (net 7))
 (segment (start 178.899 45.101) (end 167.101 45.101) (width 0.2) (layer "B.Cu") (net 7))
 (segment (start 167.101 45.101) (end 166 44) (width 0.2) (layer "B.Cu") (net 7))
 (segment (start 148.5 43.5) (end 147.299 42.299) (width 0.2) (layer "F.Cu") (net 14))
 (segment (start 144.759 42.299) (end 144.759 47.749) (width 0.2) (layer "F.Cu") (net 14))
 (segment (start 147.299 42.299) (end 144.759 42.299) (width 0.2) (layer "F.Cu") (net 14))
 (segment (start 148.5 52.092) (end 148.5 57) (width 0.2) (layer "F.Cu") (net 14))
 (segment (start 144.759 47.749) (end 148.64016 47.749) (width 0.2) (layer "F.Cu") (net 14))
 (segment (start 150.796 51.47516) (end 150.48016 51.791) (width 0.2) (layer "F.Cu") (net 14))
 (segment (start 150.796 49.90484) (end 150.796 51.47516) (width 0.2) (layer "F.Cu") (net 14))
 (segment (start 150.48016 51.791) (end 148.801 51.791) (width 0.2) (layer "F.Cu") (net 14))
 (segment (start 148.64016 47.749) (end 150.796 49.90484) (width 0.2) (layer "F.Cu") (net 14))
 (segment (start 148.801 51.791) (end 148.5 52.092) (width 0.2) (layer "F.Cu") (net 14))
 (via (at 148.5 57) (size 0.6) (drill 0.3) (layers "F.Cu" "B.Cu") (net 14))
 (segment (start 126.301529 57) (end 114.799 68.502529) (width 0.2) (layer "B.Cu") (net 14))
 (segment (start 160.511357 63.3613) (end 168.8613 63.3613) (width 0.2) (layer "B.Cu") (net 14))
 (segment (start 158.837235 61.687178) (end 160.511357 63.3613) (width 0.2) (layer "B.Cu") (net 14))
 (segment (start 116.497471 70.201) (end 125.011293 61.687178) (width 0.2) (layer "B.Cu") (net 14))
 (segment (start 115.502529 70.201) (end 116.497471 70.201) (width 0.2) (layer "B.Cu") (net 14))
 (segment (start 168.8613 63.3613) (end 169.81 64.31) (width 0.2) (layer "B.Cu") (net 14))
 (segment (start 148.5 57) (end 126.301529 57) (width 0.2) (layer "B.Cu") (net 14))
 (segment (start 114.799 69.497471) (end 115.502529 70.201) (width 0.2) (layer "B.Cu") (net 14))
 (segment (start 114.799 68.502529) (end 114.799 69.497471) (width 0.2) (layer "B.Cu") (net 14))
 (segment (start 125.011293 61.687178) (end 158.837235 61.687178) (width 0.2) (layer "B.Cu") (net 14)))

